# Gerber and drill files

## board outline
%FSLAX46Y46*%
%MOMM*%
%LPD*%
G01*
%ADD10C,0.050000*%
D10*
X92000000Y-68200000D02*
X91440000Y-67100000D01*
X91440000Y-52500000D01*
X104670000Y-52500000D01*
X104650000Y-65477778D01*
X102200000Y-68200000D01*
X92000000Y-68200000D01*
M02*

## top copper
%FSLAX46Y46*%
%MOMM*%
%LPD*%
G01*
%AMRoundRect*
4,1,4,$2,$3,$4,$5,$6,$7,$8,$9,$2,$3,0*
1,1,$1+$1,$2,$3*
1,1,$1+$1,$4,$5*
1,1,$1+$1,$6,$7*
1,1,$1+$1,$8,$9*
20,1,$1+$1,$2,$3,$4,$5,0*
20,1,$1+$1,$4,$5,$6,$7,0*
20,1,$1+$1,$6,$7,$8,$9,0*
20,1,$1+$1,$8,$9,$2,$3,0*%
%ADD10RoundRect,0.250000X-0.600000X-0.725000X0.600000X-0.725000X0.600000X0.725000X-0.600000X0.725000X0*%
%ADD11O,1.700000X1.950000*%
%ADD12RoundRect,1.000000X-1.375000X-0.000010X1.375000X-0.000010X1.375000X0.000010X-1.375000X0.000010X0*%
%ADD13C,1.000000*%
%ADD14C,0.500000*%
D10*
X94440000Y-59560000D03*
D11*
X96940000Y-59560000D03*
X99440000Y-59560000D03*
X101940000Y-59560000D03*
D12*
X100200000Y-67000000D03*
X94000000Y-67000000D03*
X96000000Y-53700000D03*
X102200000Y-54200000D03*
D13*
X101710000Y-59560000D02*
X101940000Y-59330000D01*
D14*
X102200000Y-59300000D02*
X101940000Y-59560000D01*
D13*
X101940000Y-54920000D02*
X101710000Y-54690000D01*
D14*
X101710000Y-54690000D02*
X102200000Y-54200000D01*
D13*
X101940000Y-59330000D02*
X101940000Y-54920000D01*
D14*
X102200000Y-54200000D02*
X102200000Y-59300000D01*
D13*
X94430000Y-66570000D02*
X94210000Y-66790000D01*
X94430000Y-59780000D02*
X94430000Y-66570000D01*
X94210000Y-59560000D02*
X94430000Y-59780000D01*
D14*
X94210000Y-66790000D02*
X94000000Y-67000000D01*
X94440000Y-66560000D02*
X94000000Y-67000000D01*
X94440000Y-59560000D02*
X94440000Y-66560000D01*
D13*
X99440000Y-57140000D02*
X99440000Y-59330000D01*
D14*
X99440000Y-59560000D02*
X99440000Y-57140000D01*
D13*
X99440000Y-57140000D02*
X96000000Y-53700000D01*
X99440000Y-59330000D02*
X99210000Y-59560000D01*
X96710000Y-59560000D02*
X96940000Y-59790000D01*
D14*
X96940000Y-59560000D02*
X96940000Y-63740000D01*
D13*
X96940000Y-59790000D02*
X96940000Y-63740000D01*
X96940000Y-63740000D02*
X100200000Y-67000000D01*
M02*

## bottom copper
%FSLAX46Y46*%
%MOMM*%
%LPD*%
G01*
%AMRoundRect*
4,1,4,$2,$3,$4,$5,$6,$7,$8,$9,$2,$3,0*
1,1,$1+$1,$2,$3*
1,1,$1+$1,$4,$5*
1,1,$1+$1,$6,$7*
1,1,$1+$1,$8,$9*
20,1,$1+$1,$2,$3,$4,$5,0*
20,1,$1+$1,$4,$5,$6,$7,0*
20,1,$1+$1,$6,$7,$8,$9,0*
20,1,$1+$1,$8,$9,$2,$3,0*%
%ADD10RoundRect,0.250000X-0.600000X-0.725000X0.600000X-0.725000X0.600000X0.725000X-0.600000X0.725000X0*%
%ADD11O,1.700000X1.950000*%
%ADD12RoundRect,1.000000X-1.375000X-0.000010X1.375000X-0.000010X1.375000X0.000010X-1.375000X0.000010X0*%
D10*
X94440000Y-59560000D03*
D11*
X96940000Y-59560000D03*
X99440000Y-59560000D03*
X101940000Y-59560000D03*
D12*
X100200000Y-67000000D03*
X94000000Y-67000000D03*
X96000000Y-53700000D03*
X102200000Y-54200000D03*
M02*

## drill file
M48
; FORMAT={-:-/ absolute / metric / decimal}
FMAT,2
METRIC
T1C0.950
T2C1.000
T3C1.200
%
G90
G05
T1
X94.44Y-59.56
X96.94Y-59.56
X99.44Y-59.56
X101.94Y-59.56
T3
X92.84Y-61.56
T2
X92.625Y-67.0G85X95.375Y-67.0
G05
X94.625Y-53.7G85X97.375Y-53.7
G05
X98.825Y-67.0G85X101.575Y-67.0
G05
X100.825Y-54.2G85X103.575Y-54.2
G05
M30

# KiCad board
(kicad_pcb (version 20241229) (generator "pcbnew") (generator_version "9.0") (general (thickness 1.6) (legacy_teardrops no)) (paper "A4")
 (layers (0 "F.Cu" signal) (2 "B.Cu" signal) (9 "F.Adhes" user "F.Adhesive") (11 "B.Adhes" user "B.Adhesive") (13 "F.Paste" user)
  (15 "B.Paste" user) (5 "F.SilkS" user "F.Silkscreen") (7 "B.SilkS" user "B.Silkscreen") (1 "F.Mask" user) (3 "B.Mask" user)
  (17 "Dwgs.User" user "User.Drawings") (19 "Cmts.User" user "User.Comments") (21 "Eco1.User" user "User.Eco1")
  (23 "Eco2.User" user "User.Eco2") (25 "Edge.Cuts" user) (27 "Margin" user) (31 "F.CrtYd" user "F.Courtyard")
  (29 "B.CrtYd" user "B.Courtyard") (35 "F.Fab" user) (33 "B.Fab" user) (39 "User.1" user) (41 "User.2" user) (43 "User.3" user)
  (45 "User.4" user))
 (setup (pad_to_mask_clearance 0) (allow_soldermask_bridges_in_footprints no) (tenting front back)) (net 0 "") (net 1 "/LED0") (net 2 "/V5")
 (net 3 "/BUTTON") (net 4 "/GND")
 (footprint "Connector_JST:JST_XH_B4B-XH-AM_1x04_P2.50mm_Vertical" (layer "F.Cu") (at 94.44 59.56)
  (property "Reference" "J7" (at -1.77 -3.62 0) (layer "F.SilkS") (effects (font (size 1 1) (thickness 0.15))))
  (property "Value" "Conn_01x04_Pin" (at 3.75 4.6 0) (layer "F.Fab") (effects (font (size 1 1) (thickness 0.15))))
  (pad "" np_thru_hole circle (at -1.6 2) (size 1.2 1.2) (drill 1.2) (layers "*.Cu" "*.Mask"))
  (pad "1" thru_hole roundrect (at 0 0) (size 1.7 1.95) (drill 0.95) (layers "*.Cu" "*.Mask") (remove_unused_layers no)
   (roundrect_rratio 0.147059) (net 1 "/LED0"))
  (pad "2" thru_hole oval (at 2.5 0) (size 1.7 1.95) (drill 0.95) (layers "*.Cu" "*.Mask") (remove_unused_layers no) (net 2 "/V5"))
  (pad "3" thru_hole oval (at 5 0) (size 1.7 1.95) (drill 0.95) (layers "*.Cu" "*.Mask") (remove_unused_layers no) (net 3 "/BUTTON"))
  (pad "4" thru_hole oval (at 7.5 0) (size 1.7 1.95) (drill 0.95) (layers "*.Cu" "*.Mask") (remove_unused_layers no) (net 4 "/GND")))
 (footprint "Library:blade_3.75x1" (layer "F.Cu") (at 100.2 67)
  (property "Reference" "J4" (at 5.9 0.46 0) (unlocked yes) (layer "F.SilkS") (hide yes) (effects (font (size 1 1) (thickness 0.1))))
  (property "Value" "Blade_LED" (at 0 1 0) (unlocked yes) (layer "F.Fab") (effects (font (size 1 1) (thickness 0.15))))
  (pad "1" thru_hole roundrect (at 0 0) (size 4.75 2) (drill oval 3.75 1) (layers "*.Cu" "*.Mask") (remove_unused_layers no)
   (roundrect_rratio 0.5) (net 2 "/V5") (thermal_bridge_angle 45)))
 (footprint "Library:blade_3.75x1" (layer "F.Cu") (at 94 67)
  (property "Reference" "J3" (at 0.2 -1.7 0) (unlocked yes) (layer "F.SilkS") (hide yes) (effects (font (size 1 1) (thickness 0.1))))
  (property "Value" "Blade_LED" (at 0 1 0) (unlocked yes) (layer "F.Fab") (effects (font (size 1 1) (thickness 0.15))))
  (pad "1" thru_hole roundrect (at 0 0) (size 4.75 2) (drill oval 3.75 1) (layers "*.Cu" "*.Mask") (remove_unused_layers no)
   (roundrect_rratio 0.5) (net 1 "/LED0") (thermal_bridge_angle 45)))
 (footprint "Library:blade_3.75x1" (layer "F.Cu") (at 95.4 54.3)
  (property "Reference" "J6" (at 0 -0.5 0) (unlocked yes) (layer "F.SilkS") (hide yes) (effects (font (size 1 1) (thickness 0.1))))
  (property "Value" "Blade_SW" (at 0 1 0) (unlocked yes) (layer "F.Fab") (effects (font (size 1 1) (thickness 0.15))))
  (pad "1" thru_hole roundrect (at 0.6 -0.6) (size 4.75 2) (drill oval 3.75 1) (layers "*.Cu" "*.Mask") (remove_unused_layers no)
   (roundrect_rratio 0.5) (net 3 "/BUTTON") (thermal_bridge_angle 45)))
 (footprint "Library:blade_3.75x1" (layer "F.Cu") (at 101.7 55.5)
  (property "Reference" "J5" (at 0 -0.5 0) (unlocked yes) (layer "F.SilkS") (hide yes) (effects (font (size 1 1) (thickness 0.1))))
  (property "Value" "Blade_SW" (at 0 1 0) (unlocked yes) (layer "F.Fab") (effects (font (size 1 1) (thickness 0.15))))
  (pad "1" thru_hole roundrect (at 0.5 -1.3) (size 4.75 2) (drill oval 3.75 1) (layers "*.Cu" "*.Mask") (remove_unused_layers no)
   (roundrect_rratio 0.5) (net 4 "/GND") (thermal_bridge_angle 45)))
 (gr_poly
  (pts (xy 92 68.2) (xy 91.44 67.1) (xy 91.44 52.5) (xy 104.67 52.5) (xy 104.65 65.477778) (xy 102.2 68.2))
  (stroke (width 0.05) (type solid)) (fill no) (layer "Edge.Cuts"))
 (segment (start 101.71 59.56) (end 101.94 59.33) (width 1) (layer "F.Cu") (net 4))
 (segment (start 102.2 59.3) (end 101.94 59.56) (width 0.5) (layer "F.Cu") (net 4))
 (segment (start 101.94 54.92) (end 101.71 54.69) (width 1) (layer "F.Cu") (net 4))
 (segment (start 101.71 54.69) (end 102.2 54.2) (width 0.5) (layer "F.Cu") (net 4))
 (segment (start 101.94 59.33) (end 101.94 54.92) (width 1) (layer "F.Cu") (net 4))
 (segment (start 102.2 54.2) (end 102.2 59.3) (width 0.5) (layer "F.Cu") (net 4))
 (segment (start 94.43 66.57) (end 94.21 66.79) (width 1) (layer "F.Cu") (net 1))
 (segment (start 94.43 59.78) (end 94.43 66.57) (width 1) (layer "F.Cu") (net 1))
 (segment (start 94.21 59.56) (end 94.43 59.78) (width 1) (layer "F.Cu") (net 1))
 (segment (start 94.21 66.79) (end 94 67) (width 0.5) (layer "F.Cu") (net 1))
 (segment (start 94.44 66.56) (end 94 67) (width 0.5) (layer "F.Cu") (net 1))
 (segment (start 94.44 59.56) (end 94.44 66.56) (width 0.5) (layer "F.Cu") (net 1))
 (segment (start 99.44 57.14) (end 99.44 59.33) (width 1) (layer "F.Cu") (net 3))
 (segment (start 99.44 59.56) (end 99.44 57.14) (width 0.5) (layer "F.Cu") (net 3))
 (segment (start 99.44 57.14) (end 96 53.7) (width 1) (layer "F.Cu") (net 3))
 (segment (start 99.44 59.33) (end 99.21 59.56) (width 1) (layer "F.Cu") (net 3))
 (segment (start 96.71 59.56) (end 96.94 59.79) (width 1) (layer "F.Cu") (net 2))
 (segment (start 96.94 59.56) (end 96.94 63.74) (width 0.5) (layer "F.Cu") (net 2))
 (segment (start 96.94 59.79) (end 96.94 63.74) (width 1) (layer "F.Cu") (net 2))
 (segment (start 96.94 63.74) (end 100.2 67) (width 1) (layer "F.Cu") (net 2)))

